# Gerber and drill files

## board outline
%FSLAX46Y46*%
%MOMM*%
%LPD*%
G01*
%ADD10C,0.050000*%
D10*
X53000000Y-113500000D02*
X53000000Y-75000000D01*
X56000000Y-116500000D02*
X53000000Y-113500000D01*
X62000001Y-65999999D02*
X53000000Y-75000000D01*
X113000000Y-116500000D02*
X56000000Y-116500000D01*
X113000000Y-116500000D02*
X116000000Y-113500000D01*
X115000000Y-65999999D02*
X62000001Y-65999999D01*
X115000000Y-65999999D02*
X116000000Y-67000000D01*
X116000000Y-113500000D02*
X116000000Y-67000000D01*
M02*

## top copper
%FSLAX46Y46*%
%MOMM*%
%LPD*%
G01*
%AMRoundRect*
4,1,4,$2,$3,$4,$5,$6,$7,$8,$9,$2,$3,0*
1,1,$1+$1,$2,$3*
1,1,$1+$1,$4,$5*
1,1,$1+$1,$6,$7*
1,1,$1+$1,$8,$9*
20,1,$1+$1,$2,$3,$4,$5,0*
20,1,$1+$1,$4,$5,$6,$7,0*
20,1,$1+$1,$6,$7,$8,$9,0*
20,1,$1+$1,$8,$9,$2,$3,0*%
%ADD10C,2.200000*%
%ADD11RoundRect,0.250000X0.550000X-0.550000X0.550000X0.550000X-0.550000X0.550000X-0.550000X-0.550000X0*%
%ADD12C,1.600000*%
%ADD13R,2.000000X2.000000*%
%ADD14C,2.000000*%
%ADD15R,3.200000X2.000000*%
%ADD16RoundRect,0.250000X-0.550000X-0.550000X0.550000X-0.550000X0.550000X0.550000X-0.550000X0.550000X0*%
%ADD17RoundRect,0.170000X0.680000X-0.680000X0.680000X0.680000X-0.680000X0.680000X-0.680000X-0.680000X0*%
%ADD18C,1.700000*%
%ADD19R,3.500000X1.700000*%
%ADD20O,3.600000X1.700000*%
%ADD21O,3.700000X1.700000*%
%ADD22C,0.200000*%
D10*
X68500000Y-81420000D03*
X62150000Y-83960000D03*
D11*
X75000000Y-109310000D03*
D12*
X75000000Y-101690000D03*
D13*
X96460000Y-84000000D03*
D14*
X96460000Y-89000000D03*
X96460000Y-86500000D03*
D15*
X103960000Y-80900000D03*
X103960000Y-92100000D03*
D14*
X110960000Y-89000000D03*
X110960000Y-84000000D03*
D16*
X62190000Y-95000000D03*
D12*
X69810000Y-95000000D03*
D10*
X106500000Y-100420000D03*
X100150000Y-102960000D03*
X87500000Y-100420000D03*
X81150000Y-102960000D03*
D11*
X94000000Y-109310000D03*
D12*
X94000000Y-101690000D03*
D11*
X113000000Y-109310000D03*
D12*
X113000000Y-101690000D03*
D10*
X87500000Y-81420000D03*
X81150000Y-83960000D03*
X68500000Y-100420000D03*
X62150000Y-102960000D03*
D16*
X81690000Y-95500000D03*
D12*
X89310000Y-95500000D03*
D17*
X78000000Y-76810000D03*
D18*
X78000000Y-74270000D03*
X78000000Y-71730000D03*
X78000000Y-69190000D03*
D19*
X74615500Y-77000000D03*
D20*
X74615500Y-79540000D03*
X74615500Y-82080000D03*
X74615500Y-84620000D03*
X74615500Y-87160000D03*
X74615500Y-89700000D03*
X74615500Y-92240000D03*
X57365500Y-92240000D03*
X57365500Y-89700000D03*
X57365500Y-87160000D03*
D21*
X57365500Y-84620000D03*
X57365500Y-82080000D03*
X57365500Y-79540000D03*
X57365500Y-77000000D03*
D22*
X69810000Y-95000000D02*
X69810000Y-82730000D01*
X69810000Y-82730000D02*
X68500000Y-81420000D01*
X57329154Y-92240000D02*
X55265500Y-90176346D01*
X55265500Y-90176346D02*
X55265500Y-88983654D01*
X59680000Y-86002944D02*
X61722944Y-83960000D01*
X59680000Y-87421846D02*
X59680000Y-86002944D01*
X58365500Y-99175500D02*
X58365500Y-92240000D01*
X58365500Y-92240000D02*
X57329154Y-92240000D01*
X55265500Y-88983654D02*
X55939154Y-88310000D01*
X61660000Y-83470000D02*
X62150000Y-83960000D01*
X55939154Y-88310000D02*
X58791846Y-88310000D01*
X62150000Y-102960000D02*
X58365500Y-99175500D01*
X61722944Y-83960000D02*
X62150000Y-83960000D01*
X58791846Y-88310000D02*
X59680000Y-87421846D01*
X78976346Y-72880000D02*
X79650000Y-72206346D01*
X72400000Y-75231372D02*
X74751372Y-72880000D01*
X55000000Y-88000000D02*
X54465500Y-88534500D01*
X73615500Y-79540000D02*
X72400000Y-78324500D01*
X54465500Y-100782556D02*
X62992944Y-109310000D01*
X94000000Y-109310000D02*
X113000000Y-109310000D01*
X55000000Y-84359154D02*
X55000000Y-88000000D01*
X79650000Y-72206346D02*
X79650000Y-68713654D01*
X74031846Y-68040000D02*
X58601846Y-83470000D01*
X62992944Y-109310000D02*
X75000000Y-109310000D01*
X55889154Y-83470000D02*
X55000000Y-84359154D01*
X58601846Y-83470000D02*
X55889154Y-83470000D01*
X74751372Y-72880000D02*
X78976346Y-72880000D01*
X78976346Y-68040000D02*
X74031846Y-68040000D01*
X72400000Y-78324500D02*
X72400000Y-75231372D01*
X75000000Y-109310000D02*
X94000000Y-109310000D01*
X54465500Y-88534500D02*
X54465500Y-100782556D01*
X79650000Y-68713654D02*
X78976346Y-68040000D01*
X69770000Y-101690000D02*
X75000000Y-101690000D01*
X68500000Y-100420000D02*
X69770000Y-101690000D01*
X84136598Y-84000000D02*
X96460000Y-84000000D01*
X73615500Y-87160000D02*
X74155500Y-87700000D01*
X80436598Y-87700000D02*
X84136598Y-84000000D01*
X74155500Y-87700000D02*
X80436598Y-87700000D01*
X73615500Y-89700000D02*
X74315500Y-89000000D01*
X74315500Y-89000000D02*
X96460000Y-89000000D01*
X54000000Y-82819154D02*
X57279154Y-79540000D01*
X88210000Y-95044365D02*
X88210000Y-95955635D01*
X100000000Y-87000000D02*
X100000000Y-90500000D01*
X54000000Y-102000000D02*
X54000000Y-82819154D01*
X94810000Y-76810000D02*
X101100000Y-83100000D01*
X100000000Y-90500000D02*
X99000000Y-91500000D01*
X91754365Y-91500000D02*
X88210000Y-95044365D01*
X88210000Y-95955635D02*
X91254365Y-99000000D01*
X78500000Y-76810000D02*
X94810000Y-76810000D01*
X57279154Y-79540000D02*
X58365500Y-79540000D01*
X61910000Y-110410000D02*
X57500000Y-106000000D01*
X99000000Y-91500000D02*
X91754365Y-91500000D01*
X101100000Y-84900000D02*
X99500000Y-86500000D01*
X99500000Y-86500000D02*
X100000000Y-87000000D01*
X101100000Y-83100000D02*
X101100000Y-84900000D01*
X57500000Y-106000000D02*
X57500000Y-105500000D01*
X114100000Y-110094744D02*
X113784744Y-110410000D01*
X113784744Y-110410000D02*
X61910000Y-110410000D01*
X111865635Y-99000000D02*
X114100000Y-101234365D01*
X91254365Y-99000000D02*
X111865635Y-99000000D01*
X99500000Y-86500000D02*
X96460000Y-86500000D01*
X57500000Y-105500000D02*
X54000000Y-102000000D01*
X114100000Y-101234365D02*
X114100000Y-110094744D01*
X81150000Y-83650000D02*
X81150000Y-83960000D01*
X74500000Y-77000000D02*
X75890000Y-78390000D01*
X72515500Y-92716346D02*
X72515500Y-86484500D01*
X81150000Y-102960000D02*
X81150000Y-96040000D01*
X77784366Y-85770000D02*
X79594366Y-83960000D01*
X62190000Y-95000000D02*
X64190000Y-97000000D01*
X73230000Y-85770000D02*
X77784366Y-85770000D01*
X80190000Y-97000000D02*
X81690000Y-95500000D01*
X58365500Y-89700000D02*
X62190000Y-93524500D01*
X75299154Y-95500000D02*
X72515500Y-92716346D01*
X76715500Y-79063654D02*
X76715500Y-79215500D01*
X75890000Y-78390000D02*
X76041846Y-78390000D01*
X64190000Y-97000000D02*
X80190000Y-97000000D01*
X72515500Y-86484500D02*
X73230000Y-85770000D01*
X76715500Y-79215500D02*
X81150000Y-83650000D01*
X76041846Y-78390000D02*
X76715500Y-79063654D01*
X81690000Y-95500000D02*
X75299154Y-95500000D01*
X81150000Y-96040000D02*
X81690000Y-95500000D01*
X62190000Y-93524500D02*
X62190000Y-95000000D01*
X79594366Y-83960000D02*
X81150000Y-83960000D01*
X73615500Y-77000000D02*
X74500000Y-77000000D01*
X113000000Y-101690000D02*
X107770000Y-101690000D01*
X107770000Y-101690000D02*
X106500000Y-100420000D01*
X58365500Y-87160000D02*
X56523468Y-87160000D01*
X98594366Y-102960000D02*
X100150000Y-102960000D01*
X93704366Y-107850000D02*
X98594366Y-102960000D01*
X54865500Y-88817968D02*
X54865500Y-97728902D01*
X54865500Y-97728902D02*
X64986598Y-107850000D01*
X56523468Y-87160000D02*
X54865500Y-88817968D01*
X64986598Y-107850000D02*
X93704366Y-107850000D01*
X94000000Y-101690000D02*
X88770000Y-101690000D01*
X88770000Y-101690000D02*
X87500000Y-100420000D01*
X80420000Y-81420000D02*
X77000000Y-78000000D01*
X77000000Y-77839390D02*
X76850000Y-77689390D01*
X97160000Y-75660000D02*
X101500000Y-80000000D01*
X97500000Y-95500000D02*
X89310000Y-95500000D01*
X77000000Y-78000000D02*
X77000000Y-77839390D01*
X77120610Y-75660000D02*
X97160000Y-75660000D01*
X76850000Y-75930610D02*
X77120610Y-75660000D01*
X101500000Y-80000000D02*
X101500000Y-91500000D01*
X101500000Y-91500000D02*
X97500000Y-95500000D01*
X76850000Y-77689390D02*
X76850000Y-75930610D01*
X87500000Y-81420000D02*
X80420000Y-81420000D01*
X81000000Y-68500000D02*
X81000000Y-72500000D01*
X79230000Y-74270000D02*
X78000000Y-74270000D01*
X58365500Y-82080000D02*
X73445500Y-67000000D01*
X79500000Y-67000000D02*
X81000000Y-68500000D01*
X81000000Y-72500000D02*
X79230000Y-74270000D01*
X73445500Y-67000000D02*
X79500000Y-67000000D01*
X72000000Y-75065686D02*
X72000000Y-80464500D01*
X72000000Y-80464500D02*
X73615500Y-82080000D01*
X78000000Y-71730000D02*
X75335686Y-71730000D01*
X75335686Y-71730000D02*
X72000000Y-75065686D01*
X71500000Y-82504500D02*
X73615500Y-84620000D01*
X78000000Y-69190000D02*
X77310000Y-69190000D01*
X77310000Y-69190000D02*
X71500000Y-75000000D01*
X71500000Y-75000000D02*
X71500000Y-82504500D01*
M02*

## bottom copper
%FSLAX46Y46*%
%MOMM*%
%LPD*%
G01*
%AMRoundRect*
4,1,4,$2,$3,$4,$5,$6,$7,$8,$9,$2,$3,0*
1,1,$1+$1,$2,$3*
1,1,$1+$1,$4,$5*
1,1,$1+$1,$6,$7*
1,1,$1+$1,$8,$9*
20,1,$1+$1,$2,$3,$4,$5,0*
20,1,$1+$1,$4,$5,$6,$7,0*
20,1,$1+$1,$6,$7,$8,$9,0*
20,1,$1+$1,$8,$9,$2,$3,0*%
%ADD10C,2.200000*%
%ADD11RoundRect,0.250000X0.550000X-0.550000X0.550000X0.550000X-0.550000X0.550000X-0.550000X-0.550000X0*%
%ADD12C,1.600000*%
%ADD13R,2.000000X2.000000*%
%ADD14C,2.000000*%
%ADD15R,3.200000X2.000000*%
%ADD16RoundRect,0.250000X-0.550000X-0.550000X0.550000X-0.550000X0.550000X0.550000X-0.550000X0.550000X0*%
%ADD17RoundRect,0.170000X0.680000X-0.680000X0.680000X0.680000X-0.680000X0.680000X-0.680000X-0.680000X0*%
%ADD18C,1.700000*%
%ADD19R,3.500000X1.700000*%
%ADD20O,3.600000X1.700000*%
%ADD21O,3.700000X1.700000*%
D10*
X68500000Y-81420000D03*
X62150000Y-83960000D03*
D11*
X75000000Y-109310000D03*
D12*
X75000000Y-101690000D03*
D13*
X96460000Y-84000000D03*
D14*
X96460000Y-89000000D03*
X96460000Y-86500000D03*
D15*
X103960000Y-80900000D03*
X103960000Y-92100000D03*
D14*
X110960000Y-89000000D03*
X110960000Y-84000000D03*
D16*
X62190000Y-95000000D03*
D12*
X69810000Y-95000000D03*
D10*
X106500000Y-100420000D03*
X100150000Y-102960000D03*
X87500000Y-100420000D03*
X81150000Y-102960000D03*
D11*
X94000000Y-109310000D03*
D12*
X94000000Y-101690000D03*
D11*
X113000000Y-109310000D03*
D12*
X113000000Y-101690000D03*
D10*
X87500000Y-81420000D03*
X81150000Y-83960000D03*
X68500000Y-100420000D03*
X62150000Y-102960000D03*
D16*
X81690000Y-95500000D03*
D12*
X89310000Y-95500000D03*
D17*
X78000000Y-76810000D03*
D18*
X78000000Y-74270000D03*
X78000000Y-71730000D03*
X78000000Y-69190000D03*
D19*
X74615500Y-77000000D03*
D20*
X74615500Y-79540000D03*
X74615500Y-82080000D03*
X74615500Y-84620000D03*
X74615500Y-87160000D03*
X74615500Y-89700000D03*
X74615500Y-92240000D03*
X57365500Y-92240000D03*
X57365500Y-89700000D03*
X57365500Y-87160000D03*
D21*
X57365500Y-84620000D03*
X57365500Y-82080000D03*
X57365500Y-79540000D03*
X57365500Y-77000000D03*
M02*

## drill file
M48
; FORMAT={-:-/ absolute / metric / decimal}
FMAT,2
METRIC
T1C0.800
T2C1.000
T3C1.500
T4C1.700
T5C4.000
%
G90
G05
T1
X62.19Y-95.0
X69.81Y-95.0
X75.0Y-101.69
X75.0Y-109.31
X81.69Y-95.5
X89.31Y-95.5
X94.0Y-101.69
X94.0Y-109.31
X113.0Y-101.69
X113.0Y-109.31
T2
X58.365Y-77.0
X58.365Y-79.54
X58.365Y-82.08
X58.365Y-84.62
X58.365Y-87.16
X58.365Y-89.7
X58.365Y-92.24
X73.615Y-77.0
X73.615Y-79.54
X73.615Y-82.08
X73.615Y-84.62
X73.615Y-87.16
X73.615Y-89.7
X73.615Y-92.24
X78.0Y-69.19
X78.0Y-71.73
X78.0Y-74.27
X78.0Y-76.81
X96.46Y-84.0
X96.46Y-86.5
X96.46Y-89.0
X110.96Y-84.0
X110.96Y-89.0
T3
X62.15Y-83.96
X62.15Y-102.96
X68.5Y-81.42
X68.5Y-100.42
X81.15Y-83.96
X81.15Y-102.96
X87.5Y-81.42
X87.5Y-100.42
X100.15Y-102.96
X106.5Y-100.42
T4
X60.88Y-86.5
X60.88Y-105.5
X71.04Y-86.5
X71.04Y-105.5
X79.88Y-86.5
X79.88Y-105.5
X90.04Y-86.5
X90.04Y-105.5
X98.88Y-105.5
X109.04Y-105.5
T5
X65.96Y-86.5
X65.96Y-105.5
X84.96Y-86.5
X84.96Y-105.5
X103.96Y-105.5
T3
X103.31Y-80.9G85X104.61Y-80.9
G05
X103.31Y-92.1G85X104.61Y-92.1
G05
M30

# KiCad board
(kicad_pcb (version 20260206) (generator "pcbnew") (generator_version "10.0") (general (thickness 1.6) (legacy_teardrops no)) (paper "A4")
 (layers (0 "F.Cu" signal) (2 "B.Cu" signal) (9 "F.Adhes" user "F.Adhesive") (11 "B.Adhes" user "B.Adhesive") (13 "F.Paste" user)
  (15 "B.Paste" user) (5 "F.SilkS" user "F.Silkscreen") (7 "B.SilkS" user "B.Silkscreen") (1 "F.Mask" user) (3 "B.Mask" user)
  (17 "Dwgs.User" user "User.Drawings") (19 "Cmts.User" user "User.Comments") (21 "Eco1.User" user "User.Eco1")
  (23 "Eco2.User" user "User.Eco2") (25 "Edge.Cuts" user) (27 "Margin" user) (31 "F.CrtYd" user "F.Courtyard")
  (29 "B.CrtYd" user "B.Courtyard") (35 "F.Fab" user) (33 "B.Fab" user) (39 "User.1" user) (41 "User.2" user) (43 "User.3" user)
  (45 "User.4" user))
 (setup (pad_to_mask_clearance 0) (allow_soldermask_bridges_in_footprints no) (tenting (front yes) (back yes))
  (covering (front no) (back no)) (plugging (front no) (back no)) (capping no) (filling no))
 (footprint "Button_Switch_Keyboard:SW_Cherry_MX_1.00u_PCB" (layer "F.Cu") (at 68.5 81.42)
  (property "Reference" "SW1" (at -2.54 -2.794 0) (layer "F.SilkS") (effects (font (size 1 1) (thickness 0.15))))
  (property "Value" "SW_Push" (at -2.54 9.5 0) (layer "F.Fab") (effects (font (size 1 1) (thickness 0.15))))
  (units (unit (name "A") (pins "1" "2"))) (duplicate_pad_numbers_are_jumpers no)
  (pad "" np_thru_hole circle (at -7.62 5.08) (size 1.7 1.7) (drill 1.7) (layers "*.Cu" "*.Mask"))
  (pad "" np_thru_hole circle (at -2.54 5.08) (size 4 4) (drill 4) (layers "*.Cu" "*.Mask"))
  (pad "" np_thru_hole circle (at 2.54 5.08) (size 1.7 1.7) (drill 1.7) (layers "*.Cu" "*.Mask"))
  (pad "1" thru_hole circle (at 0 0) (size 2.2 2.2) (drill 1.5) (layers "*.Cu" "*.Mask") (remove_unused_layers no) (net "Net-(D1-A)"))
  (pad "2" thru_hole circle (at -6.35 2.54) (size 2.2 2.2) (drill 1.5) (layers "*.Cu" "*.Mask") (remove_unused_layers no) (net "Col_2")))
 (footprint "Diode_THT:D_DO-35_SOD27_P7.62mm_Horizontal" (layer "F.Cu") (at 75 109.31 90)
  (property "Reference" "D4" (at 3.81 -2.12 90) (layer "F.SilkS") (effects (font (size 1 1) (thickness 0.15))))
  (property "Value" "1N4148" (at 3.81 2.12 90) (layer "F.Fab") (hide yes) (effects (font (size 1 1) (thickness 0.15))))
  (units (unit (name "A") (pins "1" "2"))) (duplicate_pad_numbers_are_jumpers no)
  (pad "1" thru_hole roundrect (at 0 0 90) (size 1.6 1.6) (drill 0.8) (layers "*.Cu" "*.Mask") (remove_unused_layers no)
   (roundrect_rratio 0.15625) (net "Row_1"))
  (pad "2" thru_hole circle (at 7.62 0 90) (size 1.6 1.6) (drill 0.8) (layers "*.Cu" "*.Mask") (remove_unused_layers no) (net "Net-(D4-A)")))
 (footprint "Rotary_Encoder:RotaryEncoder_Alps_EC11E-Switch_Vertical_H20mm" (layer "F.Cu") (at 96.46 84)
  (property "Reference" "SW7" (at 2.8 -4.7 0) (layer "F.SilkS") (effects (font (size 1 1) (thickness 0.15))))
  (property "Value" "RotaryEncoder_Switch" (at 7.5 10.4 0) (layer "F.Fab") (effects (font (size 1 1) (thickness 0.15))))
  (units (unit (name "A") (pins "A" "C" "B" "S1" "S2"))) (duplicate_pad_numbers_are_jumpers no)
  (pad "A" thru_hole rect (at 0 0) (size 2 2) (drill 1) (layers "*.Cu" "*.Mask") (remove_unused_layers no) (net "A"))
  (pad "B" thru_hole circle (at 0 5) (size 2 2) (drill 1) (layers "*.Cu" "*.Mask") (remove_unused_layers no) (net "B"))
  (pad "C" thru_hole circle (at 0 2.5) (size 2 2) (drill 1) (layers "*.Cu" "*.Mask") (remove_unused_layers no) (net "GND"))
  (pad "MP" thru_hole rect (at 7.5 -3.1) (size 3.2 2) (drill oval 2.8 1.5) (layers "*.Cu" "*.Mask") (remove_unused_layers no))
  (pad "MP" thru_hole rect (at 7.5 8.1) (size 3.2 2) (drill oval 2.8 1.5) (layers "*.Cu" "*.Mask") (remove_unused_layers no))
  (pad "S1" thru_hole circle (at 14.5 5) (size 2 2) (drill 1) (layers "*.Cu" "*.Mask") (remove_unused_layers no)
   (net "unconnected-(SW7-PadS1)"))
  (pad "S2" thru_hole circle (at 14.5 0) (size 2 2) (drill 1) (layers "*.Cu" "*.Mask") (remove_unused_layers no)
   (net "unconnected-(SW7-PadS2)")))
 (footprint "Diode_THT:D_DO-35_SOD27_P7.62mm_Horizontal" (layer "F.Cu") (at 62.19 95)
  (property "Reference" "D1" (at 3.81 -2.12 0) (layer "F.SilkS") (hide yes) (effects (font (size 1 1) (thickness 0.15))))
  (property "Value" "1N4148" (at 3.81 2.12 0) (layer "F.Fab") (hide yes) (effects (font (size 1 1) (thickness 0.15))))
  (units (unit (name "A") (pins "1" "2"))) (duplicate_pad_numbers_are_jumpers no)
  (pad "1" thru_hole roundrect (at 0 0) (size 1.6 1.6) (drill 0.8) (layers "*.Cu" "*.Mask") (remove_unused_layers no)
   (roundrect_rratio 0.15625) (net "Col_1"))
  (pad "2" thru_hole circle (at 7.62 0) (size 1.6 1.6) (drill 0.8) (layers "*.Cu" "*.Mask") (remove_unused_layers no) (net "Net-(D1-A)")))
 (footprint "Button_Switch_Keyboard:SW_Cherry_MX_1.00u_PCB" (layer "F.Cu") (at 106.5 100.42)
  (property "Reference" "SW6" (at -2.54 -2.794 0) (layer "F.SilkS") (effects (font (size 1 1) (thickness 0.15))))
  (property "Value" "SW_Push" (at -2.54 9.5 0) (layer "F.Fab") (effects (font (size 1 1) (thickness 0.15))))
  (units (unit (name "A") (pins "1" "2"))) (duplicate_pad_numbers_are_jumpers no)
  (pad "" np_thru_hole circle (at -7.62 5.08) (size 1.7 1.7) (drill 1.7) (layers "*.Cu" "*.Mask"))
  (pad "" np_thru_hole circle (at -2.54 5.08) (size 4 4) (drill 4) (layers "*.Cu" "*.Mask"))
  (pad "" np_thru_hole circle (at 2.54 5.08) (size 1.7 1.7) (drill 1.7) (layers "*.Cu" "*.Mask"))
  (pad "1" thru_hole circle (at 0 0) (size 2.2 2.2) (drill 1.5) (layers "*.Cu" "*.Mask") (remove_unused_layers no) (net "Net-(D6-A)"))
  (pad "2" thru_hole circle (at -6.35 2.54) (size 2.2 2.2) (drill 1.5) (layers "*.Cu" "*.Mask") (remove_unused_layers no) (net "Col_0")))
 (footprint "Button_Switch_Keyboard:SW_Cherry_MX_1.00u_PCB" (layer "F.Cu") (at 87.5 100.42)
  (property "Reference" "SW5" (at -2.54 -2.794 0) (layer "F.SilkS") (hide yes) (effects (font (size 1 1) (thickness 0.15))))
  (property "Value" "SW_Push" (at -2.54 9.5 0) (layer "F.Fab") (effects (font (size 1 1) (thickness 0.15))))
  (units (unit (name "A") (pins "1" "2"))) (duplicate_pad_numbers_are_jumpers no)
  (pad "" np_thru_hole circle (at -7.62 5.08) (size 1.7 1.7) (drill 1.7) (layers "*.Cu" "*.Mask"))
  (pad "" np_thru_hole circle (at -2.54 5.08) (size 4 4) (drill 4) (layers "*.Cu" "*.Mask"))
  (pad "" np_thru_hole circle (at 2.54 5.08) (size 1.7 1.7) (drill 1.7) (layers "*.Cu" "*.Mask"))
  (pad "1" thru_hole circle (at 0 0) (size 2.2 2.2) (drill 1.5) (layers "*.Cu" "*.Mask") (remove_unused_layers no) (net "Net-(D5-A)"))
  (pad "2" thru_hole circle (at -6.35 2.54) (size 2.2 2.2) (drill 1.5) (layers "*.Cu" "*.Mask") (remove_unused_layers no) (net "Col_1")))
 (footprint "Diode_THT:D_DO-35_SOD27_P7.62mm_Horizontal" (layer "F.Cu") (at 94 109.31 90)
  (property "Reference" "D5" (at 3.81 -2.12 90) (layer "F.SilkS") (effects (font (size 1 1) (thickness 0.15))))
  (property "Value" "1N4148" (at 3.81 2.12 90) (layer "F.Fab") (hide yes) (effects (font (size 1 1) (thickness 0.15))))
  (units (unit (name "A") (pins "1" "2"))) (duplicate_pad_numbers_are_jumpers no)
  (pad "1" thru_hole roundrect (at 0 0 90) (size 1.6 1.6) (drill 0.8) (layers "*.Cu" "*.Mask") (remove_unused_layers no)
   (roundrect_rratio 0.15625) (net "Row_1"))
  (pad "2" thru_hole circle (at 7.62 0 90) (size 1.6 1.6) (drill 0.8) (layers "*.Cu" "*.Mask") (remove_unused_layers no) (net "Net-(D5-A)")))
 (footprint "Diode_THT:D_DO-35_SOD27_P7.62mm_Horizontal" (layer "F.Cu") (at 113 109.31 90)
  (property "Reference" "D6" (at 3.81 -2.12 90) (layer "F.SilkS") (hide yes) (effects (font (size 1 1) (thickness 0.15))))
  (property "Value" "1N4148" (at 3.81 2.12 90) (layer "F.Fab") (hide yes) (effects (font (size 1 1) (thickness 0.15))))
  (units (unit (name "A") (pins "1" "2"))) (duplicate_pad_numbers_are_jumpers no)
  (pad "1" thru_hole roundrect (at 0 0 90) (size 1.6 1.6) (drill 0.8) (layers "*.Cu" "*.Mask") (remove_unused_layers no)
   (roundrect_rratio 0.15625) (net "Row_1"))
  (pad "2" thru_hole circle (at 7.62 0 90) (size 1.6 1.6) (drill 0.8) (layers "*.Cu" "*.Mask") (remove_unused_layers no) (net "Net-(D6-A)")))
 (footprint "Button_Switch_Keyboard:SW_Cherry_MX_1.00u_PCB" (layer "F.Cu") (at 87.5 81.42)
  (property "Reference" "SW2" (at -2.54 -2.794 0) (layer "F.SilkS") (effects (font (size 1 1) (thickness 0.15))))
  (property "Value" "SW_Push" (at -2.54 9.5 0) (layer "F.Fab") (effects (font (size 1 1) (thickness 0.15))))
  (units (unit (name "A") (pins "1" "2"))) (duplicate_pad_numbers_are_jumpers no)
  (pad "" np_thru_hole circle (at -7.62 5.08) (size 1.7 1.7) (drill 1.7) (layers "*.Cu" "*.Mask"))
  (pad "" np_thru_hole circle (at -2.54 5.08) (size 4 4) (drill 4) (layers "*.Cu" "*.Mask"))
  (pad "" np_thru_hole circle (at 2.54 5.08) (size 1.7 1.7) (drill 1.7) (layers "*.Cu" "*.Mask"))
  (pad "1" thru_hole circle (at 0 0) (size 2.2 2.2) (drill 1.5) (layers "*.Cu" "*.Mask") (remove_unused_layers no) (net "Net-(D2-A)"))
  (pad "2" thru_hole circle (at -6.35 2.54) (size 2.2 2.2) (drill 1.5) (layers "*.Cu" "*.Mask") (remove_unused_layers no) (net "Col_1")))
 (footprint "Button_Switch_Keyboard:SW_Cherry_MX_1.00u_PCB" (layer "F.Cu") (at 68.5 100.42)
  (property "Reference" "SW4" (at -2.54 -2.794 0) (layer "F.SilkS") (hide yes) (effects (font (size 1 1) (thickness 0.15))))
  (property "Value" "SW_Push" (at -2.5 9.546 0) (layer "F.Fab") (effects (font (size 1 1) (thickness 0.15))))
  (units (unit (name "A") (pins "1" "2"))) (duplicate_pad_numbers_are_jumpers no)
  (pad "" np_thru_hole circle (at -7.62 5.08) (size 1.7 1.7) (drill 1.7) (layers "*.Cu" "*.Mask"))
  (pad "" np_thru_hole circle (at -2.54 5.08) (size 4 4) (drill 4) (layers "*.Cu" "*.Mask"))
  (pad "" np_thru_hole circle (at 2.54 5.08) (size 1.7 1.7) (drill 1.7) (layers "*.Cu" "*.Mask"))
  (pad "1" thru_hole circle (at 0 0) (size 2.2 2.2) (drill 1.5) (layers "*.Cu" "*.Mask") (remove_unused_layers no) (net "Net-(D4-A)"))
  (pad "2" thru_hole circle (at -6.35 2.54) (size 2.2 2.2) (drill 1.5) (layers "*.Cu" "*.Mask") (remove_unused_layers no) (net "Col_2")))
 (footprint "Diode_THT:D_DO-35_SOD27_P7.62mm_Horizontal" (layer "F.Cu") (at 81.69 95.5)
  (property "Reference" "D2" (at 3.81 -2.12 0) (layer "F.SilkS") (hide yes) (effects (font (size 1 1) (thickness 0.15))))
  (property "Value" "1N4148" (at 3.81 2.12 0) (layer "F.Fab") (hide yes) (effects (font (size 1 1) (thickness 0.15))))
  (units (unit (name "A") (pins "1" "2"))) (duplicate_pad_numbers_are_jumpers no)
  (pad "1" thru_hole roundrect (at 0 0) (size 1.6 1.6) (drill 0.8) (layers "*.Cu" "*.Mask") (remove_unused_layers no)
   (roundrect_rratio 0.15625) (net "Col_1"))
  (pad "2" thru_hole circle (at 7.62 0) (size 1.6 1.6) (drill 0.8) (layers "*.Cu" "*.Mask") (remove_unused_layers no) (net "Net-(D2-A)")))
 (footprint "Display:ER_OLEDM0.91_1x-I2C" (layer "F.Cu") (at 78 76.81 90)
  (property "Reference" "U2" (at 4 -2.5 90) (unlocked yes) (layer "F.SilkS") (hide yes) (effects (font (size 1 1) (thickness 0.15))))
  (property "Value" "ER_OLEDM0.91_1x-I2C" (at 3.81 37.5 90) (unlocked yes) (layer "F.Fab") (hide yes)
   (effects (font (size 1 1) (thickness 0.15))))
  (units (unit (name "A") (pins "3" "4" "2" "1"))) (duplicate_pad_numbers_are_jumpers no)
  (pad "1" thru_hole roundrect (at 0 0 90) (size 1.7 1.7) (drill 1) (layers "*.Cu" "*.Mask") (remove_unused_layers no)
   (roundrect_rratio 0.1) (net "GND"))
  (pad "2" thru_hole circle (at 2.54 0 90) (size 1.7 1.7) (drill 1) (layers "*.Cu" "*.Mask") (remove_unused_layers no) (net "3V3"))
  (pad "3" thru_hole circle (at 5.08 0 90) (size 1.7 1.7) (drill 1) (layers "*.Cu" "*.Mask") (remove_unused_layers no) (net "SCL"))
  (pad "4" thru_hole circle (at 7.62 0 90) (size 1.7 1.7) (drill 1) (layers "*.Cu" "*.Mask") (remove_unused_layers no) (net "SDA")))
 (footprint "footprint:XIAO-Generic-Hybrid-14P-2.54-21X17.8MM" (layer "B.Cu") (at 65.9905 84.62 180)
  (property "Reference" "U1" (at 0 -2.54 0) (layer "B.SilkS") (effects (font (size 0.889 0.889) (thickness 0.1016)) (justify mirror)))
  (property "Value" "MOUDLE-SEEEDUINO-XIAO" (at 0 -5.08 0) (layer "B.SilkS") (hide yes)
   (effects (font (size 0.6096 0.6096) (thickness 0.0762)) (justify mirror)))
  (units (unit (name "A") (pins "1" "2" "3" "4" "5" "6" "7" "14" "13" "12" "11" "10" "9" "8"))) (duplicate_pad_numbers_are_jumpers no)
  (pad "1" thru_hole rect (at -7.625 7.62 180) (size 3.5 1.7) (drill 1 (offset -1 0)) (layers "*.Cu" "*.Mask") (remove_unused_layers no)
   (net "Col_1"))
  (pad "2" thru_hole oval (at -7.625 5.08 180) (size 3.6 1.7) (drill 1 (offset -1 0)) (layers "*.Cu" "*.Mask") (remove_unused_layers no)
   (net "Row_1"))
  (pad "3" thru_hole oval (at -7.625 2.54 180) (size 3.6 1.7) (drill 1 (offset -1 0)) (layers "*.Cu" "*.Mask") (remove_unused_layers no)
   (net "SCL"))
  (pad "4" thru_hole oval (at -7.625 0 180) (size 3.6 1.7) (drill 1 (offset -1 0)) (layers "*.Cu" "*.Mask") (remove_unused_layers no)
   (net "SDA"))
  (pad "5" thru_hole oval (at -7.625 -2.54 180) (size 3.6 1.7) (drill 1 (offset -1 0)) (layers "*.Cu" "*.Mask") (remove_unused_layers no)
   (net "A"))
  (pad "6" thru_hole oval (at -7.625 -5.08) (size 3.6 1.7) (drill 1 (offset 1 0)) (layers "*.Cu" "*.Mask") (remove_unused_layers no)
   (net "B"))
  (pad "7" thru_hole oval (at -7.625 -7.62 180) (size 3.6 1.7) (drill 1 (offset -1 0)) (layers "*.Cu" "*.Mask") (remove_unused_layers no)
   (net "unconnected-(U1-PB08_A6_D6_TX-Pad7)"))
  (pad "8" thru_hole oval (at 7.625 -7.62 180) (size 3.6 1.7) (drill 1 (offset 1 0)) (layers "*.Cu" "*.Mask") (remove_unused_layers no)
   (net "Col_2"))
  (pad "9" thru_hole oval (at 7.625 -5.08 180) (size 3.6 1.7) (drill 1 (offset 1 0)) (layers "*.Cu" "*.Mask") (remove_unused_layers no)
   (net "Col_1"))
  (pad "10" thru_hole oval (at 7.625 -2.54 180) (size 3.6 1.7) (drill 1 (offset 1 0)) (layers "*.Cu" "*.Mask") (remove_unused_layers no)
   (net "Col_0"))
  (pad "11" thru_hole oval (at 7.625 0 180) (size 3.7 1.7) (drill 1 (offset 1 0)) (layers "*.Cu" "*.Mask") (remove_unused_layers no)
   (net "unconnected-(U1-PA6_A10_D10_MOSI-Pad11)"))
  (pad "12" thru_hole oval (at 7.625 2.54 180) (size 3.7 1.7) (drill 1 (offset 1 0)) (layers "*.Cu" "*.Mask") (remove_unused_layers no)
   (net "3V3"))
  (pad "13" thru_hole oval (at 7.625 5.08 180) (size 3.7 1.7) (drill 1 (offset 1 0)) (layers "*.Cu" "*.Mask") (remove_unused_layers no)
   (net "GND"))
  (pad "14" thru_hole oval (at 7.625 7.62 180) (size 3.7 1.7) (drill 1 (offset 1 0)) (layers "*.Cu" "*.Mask") (remove_unused_layers no)
   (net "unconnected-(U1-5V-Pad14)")))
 (gr_line (start 53 113.5) (end 53 75) (stroke (width 0.05) (type default)) (layer "Edge.Cuts"))
 (gr_line (start 56 116.5) (end 53 113.5) (stroke (width 0.05) (type default)) (layer "Edge.Cuts"))
 (gr_line (start 62.000001 65.999999) (end 53 75) (stroke (width 0.05) (type default)) (layer "Edge.Cuts"))
 (gr_line (start 113 116.5) (end 56 116.5) (stroke (width 0.05) (type default)) (layer "Edge.Cuts"))
 (gr_line (start 113 116.5) (end 116 113.5) (stroke (width 0.05) (type default)) (layer "Edge.Cuts"))
 (gr_line (start 115 65.999999) (end 62.000001 65.999999) (stroke (width 0.05) (type default)) (layer "Edge.Cuts"))
 (gr_line (start 115 65.999999) (end 116 67) (stroke (width 0.05) (type default)) (layer "Edge.Cuts"))
 (gr_line (start 116 113.5) (end 116 67) (stroke (width 0.05) (type default)) (layer "Edge.Cuts"))
 (segment (start 69.81 95) (end 69.81 82.73) (width 0.2) (layer "F.Cu") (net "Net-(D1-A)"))
 (segment (start 69.81 82.73) (end 68.5 81.42) (width 0.2) (layer "F.Cu") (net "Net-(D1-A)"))
 (segment (start 57.329154 92.24) (end 55.2655 90.176346) (width 0.2) (layer "F.Cu") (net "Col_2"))
 (segment (start 55.2655 90.176346) (end 55.2655 88.983654) (width 0.2) (layer "F.Cu") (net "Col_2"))
 (segment (start 59.68 86.002944) (end 61.722944 83.96) (width 0.2) (layer "F.Cu") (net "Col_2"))
 (segment (start 59.68 87.421846) (end 59.68 86.002944) (width 0.2) (layer "F.Cu") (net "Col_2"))
 (segment (start 58.3655 99.1755) (end 58.3655 92.24) (width 0.2) (layer "F.Cu") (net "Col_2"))
 (segment (start 58.3655 92.24) (end 57.329154 92.24) (width 0.2) (layer "F.Cu") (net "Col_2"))
 (segment (start 55.2655 88.983654) (end 55.939154 88.31) (width 0.2) (layer "F.Cu") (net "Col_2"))
 (segment (start 61.66 83.47) (end 62.15 83.96) (width 0.2) (layer "F.Cu") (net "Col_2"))
 (segment (start 55.939154 88.31) (end 58.791846 88.31) (width 0.2) (layer "F.Cu") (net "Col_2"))
 (segment (start 62.15 102.96) (end 58.3655 99.1755) (width 0.2) (layer "F.Cu") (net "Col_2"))
 (segment (start 61.722944 83.96) (end 62.15 83.96) (width 0.2) (layer "F.Cu") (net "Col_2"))
 (segment (start 58.791846 88.31) (end 59.68 87.421846) (width 0.2) (layer "F.Cu") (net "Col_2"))
 (segment (start 78.976346 72.88) (end 79.65 72.206346) (width 0.2) (layer "F.Cu") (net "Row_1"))
 (segment (start 72.4 75.231372) (end 74.751372 72.88) (width 0.2) (layer "F.Cu") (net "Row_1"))
 (segment (start 55 88) (end 54.4655 88.5345) (width 0.2) (layer "F.Cu") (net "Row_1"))
 (segment (start 73.6155 79.54) (end 72.4 78.3245) (width 0.2) (layer "F.Cu") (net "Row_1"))
 (segment (start 54.4655 100.782556) (end 62.992944 109.31) (width 0.2) (layer "F.Cu") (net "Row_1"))
 (segment (start 94 109.31) (end 113 109.31) (width 0.2) (layer "F.Cu") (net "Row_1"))
 (segment (start 55 84.359154) (end 55 88) (width 0.2) (layer "F.Cu") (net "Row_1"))
 (segment (start 79.65 72.206346) (end 79.65 68.713654) (width 0.2) (layer "F.Cu") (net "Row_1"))
 (segment (start 74.031846 68.04) (end 58.601846 83.47) (width 0.2) (layer "F.Cu") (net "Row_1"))
 (segment (start 62.992944 109.31) (end 75 109.31) (width 0.2) (layer "F.Cu") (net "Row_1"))
 (segment (start 55.889154 83.47) (end 55 84.359154) (width 0.2) (layer "F.Cu") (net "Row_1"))
 (segment (start 58.601846 83.47) (end 55.889154 83.47) (width 0.2) (layer "F.Cu") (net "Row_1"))
 (segment (start 74.751372 72.88) (end 78.976346 72.88) (width 0.2) (layer "F.Cu") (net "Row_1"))
 (segment (start 78.976346 68.04) (end 74.031846 68.04) (width 0.2) (layer "F.Cu") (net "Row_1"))
 (segment (start 72.4 78.3245) (end 72.4 75.231372) (width 0.2) (layer "F.Cu") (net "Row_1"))
 (segment (start 75 109.31) (end 94 109.31) (width 0.2) (layer "F.Cu") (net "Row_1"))
 (segment (start 54.4655 88.5345) (end 54.4655 100.782556) (width 0.2) (layer "F.Cu") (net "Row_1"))
 (segment (start 79.65 68.713654) (end 78.976346 68.04) (width 0.2) (layer "F.Cu") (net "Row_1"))
 (segment (start 69.77 101.69) (end 75 101.69) (width 0.2) (layer "F.Cu") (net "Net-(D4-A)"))
 (segment (start 68.5 100.42) (end 69.77 101.69) (width 0.2) (layer "F.Cu") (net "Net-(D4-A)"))
 (segment (start 84.136598 84) (end 96.46 84) (width 0.2) (layer "F.Cu") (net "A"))
 (segment (start 73.6155 87.16) (end 74.1555 87.7) (width 0.2) (layer "F.Cu") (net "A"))
 (segment (start 80.436598 87.7) (end 84.136598 84) (width 0.2) (layer "F.Cu") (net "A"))
 (segment (start 74.1555 87.7) (end 80.436598 87.7) (width 0.2) (layer "F.Cu") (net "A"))
 (segment (start 73.6155 89.7) (end 74.3155 89) (width 0.2) (layer "F.Cu") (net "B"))
 (segment (start 74.3155 89) (end 96.46 89) (width 0.2) (layer "F.Cu") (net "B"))
 (segment (start 54 82.819154) (end 57.279154 79.54) (width 0.2) (layer "F.Cu") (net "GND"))
 (segment (start 88.21 95.044365) (end 88.21 95.955635) (width 0.2) (layer "F.Cu") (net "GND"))
 (segment (start 100 87) (end 100 90.5) (width 0.2) (layer "F.Cu") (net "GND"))
 (segment (start 54 102) (end 54 82.819154) (width 0.2) (layer "F.Cu") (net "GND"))
 (segment (start 94.81 76.81) (end 101.1 83.1) (width 0.2) (layer "F.Cu") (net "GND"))
 (segment (start 100 90.5) (end 99 91.5) (width 0.2) (layer "F.Cu") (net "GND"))
 (segment (start 91.754365 91.5) (end 88.21 95.044365) (width 0.2) (layer "F.Cu") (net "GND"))
 (segment (start 88.21 95.955635) (end 91.254365 99) (width 0.2) (layer "F.Cu") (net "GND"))
 (segment (start 78.5 76.81) (end 94.81 76.81) (width 0.2) (layer "F.Cu") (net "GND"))
 (segment (start 57.279154 79.54) (end 58.3655 79.54) (width 0.2) (layer "F.Cu") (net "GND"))
 (segment (start 61.91 110.41) (end 57.5 106) (width 0.2) (layer "F.Cu") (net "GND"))
 (segment (start 99 91.5) (end 91.754365 91.5) (width 0.2) (layer "F.Cu") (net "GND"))
 (segment (start 101.1 84.9) (end 99.5 86.5) (width 0.2) (layer "F.Cu") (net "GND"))
 (segment (start 99.5 86.5) (end 100 87) (width 0.2) (layer "F.Cu") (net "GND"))
 (segment (start 101.1 83.1) (end 101.1 84.9) (width 0.2) (layer "F.Cu") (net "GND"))
 (segment (start 57.5 106) (end 57.5 105.5) (width 0.2) (layer "F.Cu") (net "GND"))
 (segment (start 114.1 110.094744) (end 113.784744 110.41) (width 0.2) (layer "F.Cu") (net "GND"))
 (segment (start 113.784744 110.41) (end 61.91 110.41) (width 0.2) (layer "F.Cu") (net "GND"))
 (segment (start 111.865635 99) (end 114.1 101.234365) (width 0.2) (layer "F.Cu") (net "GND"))
 (segment (start 91.254365 99) (end 111.865635 99) (width 0.2) (layer "F.Cu") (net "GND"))
 (segment (start 99.5 86.5) (end 96.46 86.5) (width 0.2) (layer "F.Cu") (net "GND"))
 (segment (start 57.5 105.5) (end 54 102) (width 0.2) (layer "F.Cu") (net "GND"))
 (segment (start 114.1 101.234365) (end 114.1 110.094744) (width 0.2) (layer "F.Cu") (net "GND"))
 (segment (start 81.15 83.65) (end 81.15 83.96) (width 0.2) (layer "F.Cu") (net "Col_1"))
 (segment (start 74.5 77) (end 75.89 78.39) (width 0.2) (layer "F.Cu") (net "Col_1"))
 (segment (start 72.5155 92.716346) (end 72.5155 86.4845) (width 0.2) (layer "F.Cu") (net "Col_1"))
 (segment (start 81.15 102.96) (end 81.15 96.04) (width 0.2) (layer "F.Cu") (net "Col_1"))
 (segment (start 77.784366 85.77) (end 79.594366 83.96) (width 0.2) (layer "F.Cu") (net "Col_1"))
 (segment (start 62.19 95) (end 64.19 97) (width 0.2) (layer "F.Cu") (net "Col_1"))
 (segment (start 73.23 85.77) (end 77.784366 85.77) (width 0.2) (layer "F.Cu") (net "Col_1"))
 (segment (start 80.19 97) (end 81.69 95.5) (width 0.2) (layer "F.Cu") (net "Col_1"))
 (segment (start 58.3655 89.7) (end 62.19 93.5245) (width 0.2) (layer "F.Cu") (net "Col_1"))
 (segment (start 75.299154 95.5) (end 72.5155 92.716346) (width 0.2) (layer "F.Cu") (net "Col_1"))
 (segment (start 76.7155 79.063654) (end 76.7155 79.2155) (width 0.2) (layer "F.Cu") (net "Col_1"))
 (segment (start 75.89 78.39) (end 76.041846 78.39) (width 0.2) (layer "F.Cu") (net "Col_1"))
 (segment (start 64.19 97) (end 80.19 97) (width 0.2) (layer "F.Cu") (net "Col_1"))
 (segment (start 72.5155 86.4845) (end 73.23 85.77) (width 0.2) (layer "F.Cu") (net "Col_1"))
 (segment (start 76.7155 79.2155) (end 81.15 83.65) (width 0.2) (layer "F.Cu") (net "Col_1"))
 (segment (start 76.041846 78.39) (end 76.7155 79.063654) (width 0.2) (layer "F.Cu") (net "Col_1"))
 (segment (start 81.69 95.5) (end 75.299154 95.5) (width 0.2) (layer "F.Cu") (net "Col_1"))
 (segment (start 81.15 96.04) (end 81.69 95.5) (width 0.2) (layer "F.Cu") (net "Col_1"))
 (segment (start 62.19 93.5245) (end 62.19 95) (width 0.2) (layer "F.Cu") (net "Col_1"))
 (segment (start 79.594366 83.96) (end 81.15 83.96) (width 0.2) (layer "F.Cu") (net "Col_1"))
 (segment (start 73.6155 77) (end 74.5 77) (width 0.2) (layer "F.Cu") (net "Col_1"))
 (segment (start 113 101.69) (end 107.77 101.69) (width 0.2) (layer "F.Cu") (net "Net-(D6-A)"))
 (segment (start 107.77 101.69) (end 106.5 100.42) (width 0.2) (layer "F.Cu") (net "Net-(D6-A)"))
 (segment (start 58.3655 87.16) (end 56.523468 87.16) (width 0.2) (layer "F.Cu") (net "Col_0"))
 (segment (start 98.594366 102.96) (end 100.15 102.96) (width 0.2) (layer "F.Cu") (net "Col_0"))
 (segment (start 93.704366 107.85) (end 98.594366 102.96) (width 0.2) (layer "F.Cu") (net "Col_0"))
 (segment (start 54.8655 88.817968) (end 54.8655 97.728902) (width 0.2) (layer "F.Cu") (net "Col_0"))
 (segment (start 54.8655 97.728902) (end 64.986598 107.85) (width 0.2) (layer "F.Cu") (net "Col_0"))
 (segment (start 56.523468 87.16) (end 54.8655 88.817968) (width 0.2) (layer "F.Cu") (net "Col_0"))
 (segment (start 64.986598 107.85) (end 93.704366 107.85) (width 0.2) (layer "F.Cu") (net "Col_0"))
 (segment (start 94 101.69) (end 88.77 101.69) (width 0.2) (layer "F.Cu") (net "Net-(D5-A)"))
 (segment (start 88.77 101.69) (end 87.5 100.42) (width 0.2) (layer "F.Cu") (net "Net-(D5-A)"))
 (segment (start 80.42 81.42) (end 77 78) (width 0.2) (layer "F.Cu") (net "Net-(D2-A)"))
 (segment (start 77 77.83939) (end 76.85 77.68939) (width 0.2) (layer "F.Cu") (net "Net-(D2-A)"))
 (segment (start 97.16 75.66) (end 101.5 80) (width 0.2) (layer "F.Cu") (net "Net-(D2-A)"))
 (segment (start 97.5 95.5) (end 89.31 95.5) (width 0.2) (layer "F.Cu") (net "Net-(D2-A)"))
 (segment (start 77 78) (end 77 77.83939) (width 0.2) (layer "F.Cu") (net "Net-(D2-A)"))
 (segment (start 77.12061 75.66) (end 97.16 75.66) (width 0.2) (layer "F.Cu") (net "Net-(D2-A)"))
 (segment (start 76.85 75.93061) (end 77.12061 75.66) (width 0.2) (layer "F.Cu") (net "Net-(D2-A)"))
 (segment (start 101.5 80) (end 101.5 91.5) (width 0.2) (layer "F.Cu") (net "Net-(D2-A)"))
 (segment (start 101.5 91.5) (end 97.5 95.5) (width 0.2) (layer "F.Cu") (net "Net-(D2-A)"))
 (segment (start 76.85 77.68939) (end 76.85 75.93061) (width 0.2) (layer "F.Cu") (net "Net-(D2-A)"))
 (segment (start 87.5 81.42) (end 80.42 81.42) (width 0.2) (layer "F.Cu") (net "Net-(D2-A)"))
 (segment (start 81 68.5) (end 81 72.5) (width 0.2) (layer "F.Cu") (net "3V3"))
 (segment (start 79.23 74.27) (end 78 74.27) (width 0.2) (layer "F.Cu") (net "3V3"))
 (segment (start 58.3655 82.08) (end 73.4455 67) (width 0.2) (layer "F.Cu") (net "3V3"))
 (segment (start 79.5 67) (end 81 68.5) (width 0.2) (layer "F.Cu") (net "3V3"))
 (segment (start 81 72.5) (end 79.23 74.27) (width 0.2) (layer "F.Cu") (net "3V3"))
 (segment (start 73.4455 67) (end 79.5 67) (width 0.2) (layer "F.Cu") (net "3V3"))
 (segment (start 72 75.065686) (end 72 80.4645) (width 0.2) (layer "F.Cu") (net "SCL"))
 (segment (start 72 80.4645) (end 73.6155 82.08) (width 0.2) (layer "F.Cu") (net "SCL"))
 (segment (start 78 71.73) (end 75.335686 71.73) (width 0.2) (layer "F.Cu") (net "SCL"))
 (segment (start 75.335686 71.73) (end 72 75.065686) (width 0.2) (layer "F.Cu") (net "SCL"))
 (segment (start 71.5 82.5045) (end 73.6155 84.62) (width 0.2) (layer "F.Cu") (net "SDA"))
 (segment (start 78 69.19) (end 77.31 69.19) (width 0.2) (layer "F.Cu") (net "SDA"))
 (segment (start 77.31 69.19) (end 71.5 75) (width 0.2) (layer "F.Cu") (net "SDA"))
 (segment (start 71.5 75) (end 71.5 82.5045) (width 0.2) (layer "F.Cu") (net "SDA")))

